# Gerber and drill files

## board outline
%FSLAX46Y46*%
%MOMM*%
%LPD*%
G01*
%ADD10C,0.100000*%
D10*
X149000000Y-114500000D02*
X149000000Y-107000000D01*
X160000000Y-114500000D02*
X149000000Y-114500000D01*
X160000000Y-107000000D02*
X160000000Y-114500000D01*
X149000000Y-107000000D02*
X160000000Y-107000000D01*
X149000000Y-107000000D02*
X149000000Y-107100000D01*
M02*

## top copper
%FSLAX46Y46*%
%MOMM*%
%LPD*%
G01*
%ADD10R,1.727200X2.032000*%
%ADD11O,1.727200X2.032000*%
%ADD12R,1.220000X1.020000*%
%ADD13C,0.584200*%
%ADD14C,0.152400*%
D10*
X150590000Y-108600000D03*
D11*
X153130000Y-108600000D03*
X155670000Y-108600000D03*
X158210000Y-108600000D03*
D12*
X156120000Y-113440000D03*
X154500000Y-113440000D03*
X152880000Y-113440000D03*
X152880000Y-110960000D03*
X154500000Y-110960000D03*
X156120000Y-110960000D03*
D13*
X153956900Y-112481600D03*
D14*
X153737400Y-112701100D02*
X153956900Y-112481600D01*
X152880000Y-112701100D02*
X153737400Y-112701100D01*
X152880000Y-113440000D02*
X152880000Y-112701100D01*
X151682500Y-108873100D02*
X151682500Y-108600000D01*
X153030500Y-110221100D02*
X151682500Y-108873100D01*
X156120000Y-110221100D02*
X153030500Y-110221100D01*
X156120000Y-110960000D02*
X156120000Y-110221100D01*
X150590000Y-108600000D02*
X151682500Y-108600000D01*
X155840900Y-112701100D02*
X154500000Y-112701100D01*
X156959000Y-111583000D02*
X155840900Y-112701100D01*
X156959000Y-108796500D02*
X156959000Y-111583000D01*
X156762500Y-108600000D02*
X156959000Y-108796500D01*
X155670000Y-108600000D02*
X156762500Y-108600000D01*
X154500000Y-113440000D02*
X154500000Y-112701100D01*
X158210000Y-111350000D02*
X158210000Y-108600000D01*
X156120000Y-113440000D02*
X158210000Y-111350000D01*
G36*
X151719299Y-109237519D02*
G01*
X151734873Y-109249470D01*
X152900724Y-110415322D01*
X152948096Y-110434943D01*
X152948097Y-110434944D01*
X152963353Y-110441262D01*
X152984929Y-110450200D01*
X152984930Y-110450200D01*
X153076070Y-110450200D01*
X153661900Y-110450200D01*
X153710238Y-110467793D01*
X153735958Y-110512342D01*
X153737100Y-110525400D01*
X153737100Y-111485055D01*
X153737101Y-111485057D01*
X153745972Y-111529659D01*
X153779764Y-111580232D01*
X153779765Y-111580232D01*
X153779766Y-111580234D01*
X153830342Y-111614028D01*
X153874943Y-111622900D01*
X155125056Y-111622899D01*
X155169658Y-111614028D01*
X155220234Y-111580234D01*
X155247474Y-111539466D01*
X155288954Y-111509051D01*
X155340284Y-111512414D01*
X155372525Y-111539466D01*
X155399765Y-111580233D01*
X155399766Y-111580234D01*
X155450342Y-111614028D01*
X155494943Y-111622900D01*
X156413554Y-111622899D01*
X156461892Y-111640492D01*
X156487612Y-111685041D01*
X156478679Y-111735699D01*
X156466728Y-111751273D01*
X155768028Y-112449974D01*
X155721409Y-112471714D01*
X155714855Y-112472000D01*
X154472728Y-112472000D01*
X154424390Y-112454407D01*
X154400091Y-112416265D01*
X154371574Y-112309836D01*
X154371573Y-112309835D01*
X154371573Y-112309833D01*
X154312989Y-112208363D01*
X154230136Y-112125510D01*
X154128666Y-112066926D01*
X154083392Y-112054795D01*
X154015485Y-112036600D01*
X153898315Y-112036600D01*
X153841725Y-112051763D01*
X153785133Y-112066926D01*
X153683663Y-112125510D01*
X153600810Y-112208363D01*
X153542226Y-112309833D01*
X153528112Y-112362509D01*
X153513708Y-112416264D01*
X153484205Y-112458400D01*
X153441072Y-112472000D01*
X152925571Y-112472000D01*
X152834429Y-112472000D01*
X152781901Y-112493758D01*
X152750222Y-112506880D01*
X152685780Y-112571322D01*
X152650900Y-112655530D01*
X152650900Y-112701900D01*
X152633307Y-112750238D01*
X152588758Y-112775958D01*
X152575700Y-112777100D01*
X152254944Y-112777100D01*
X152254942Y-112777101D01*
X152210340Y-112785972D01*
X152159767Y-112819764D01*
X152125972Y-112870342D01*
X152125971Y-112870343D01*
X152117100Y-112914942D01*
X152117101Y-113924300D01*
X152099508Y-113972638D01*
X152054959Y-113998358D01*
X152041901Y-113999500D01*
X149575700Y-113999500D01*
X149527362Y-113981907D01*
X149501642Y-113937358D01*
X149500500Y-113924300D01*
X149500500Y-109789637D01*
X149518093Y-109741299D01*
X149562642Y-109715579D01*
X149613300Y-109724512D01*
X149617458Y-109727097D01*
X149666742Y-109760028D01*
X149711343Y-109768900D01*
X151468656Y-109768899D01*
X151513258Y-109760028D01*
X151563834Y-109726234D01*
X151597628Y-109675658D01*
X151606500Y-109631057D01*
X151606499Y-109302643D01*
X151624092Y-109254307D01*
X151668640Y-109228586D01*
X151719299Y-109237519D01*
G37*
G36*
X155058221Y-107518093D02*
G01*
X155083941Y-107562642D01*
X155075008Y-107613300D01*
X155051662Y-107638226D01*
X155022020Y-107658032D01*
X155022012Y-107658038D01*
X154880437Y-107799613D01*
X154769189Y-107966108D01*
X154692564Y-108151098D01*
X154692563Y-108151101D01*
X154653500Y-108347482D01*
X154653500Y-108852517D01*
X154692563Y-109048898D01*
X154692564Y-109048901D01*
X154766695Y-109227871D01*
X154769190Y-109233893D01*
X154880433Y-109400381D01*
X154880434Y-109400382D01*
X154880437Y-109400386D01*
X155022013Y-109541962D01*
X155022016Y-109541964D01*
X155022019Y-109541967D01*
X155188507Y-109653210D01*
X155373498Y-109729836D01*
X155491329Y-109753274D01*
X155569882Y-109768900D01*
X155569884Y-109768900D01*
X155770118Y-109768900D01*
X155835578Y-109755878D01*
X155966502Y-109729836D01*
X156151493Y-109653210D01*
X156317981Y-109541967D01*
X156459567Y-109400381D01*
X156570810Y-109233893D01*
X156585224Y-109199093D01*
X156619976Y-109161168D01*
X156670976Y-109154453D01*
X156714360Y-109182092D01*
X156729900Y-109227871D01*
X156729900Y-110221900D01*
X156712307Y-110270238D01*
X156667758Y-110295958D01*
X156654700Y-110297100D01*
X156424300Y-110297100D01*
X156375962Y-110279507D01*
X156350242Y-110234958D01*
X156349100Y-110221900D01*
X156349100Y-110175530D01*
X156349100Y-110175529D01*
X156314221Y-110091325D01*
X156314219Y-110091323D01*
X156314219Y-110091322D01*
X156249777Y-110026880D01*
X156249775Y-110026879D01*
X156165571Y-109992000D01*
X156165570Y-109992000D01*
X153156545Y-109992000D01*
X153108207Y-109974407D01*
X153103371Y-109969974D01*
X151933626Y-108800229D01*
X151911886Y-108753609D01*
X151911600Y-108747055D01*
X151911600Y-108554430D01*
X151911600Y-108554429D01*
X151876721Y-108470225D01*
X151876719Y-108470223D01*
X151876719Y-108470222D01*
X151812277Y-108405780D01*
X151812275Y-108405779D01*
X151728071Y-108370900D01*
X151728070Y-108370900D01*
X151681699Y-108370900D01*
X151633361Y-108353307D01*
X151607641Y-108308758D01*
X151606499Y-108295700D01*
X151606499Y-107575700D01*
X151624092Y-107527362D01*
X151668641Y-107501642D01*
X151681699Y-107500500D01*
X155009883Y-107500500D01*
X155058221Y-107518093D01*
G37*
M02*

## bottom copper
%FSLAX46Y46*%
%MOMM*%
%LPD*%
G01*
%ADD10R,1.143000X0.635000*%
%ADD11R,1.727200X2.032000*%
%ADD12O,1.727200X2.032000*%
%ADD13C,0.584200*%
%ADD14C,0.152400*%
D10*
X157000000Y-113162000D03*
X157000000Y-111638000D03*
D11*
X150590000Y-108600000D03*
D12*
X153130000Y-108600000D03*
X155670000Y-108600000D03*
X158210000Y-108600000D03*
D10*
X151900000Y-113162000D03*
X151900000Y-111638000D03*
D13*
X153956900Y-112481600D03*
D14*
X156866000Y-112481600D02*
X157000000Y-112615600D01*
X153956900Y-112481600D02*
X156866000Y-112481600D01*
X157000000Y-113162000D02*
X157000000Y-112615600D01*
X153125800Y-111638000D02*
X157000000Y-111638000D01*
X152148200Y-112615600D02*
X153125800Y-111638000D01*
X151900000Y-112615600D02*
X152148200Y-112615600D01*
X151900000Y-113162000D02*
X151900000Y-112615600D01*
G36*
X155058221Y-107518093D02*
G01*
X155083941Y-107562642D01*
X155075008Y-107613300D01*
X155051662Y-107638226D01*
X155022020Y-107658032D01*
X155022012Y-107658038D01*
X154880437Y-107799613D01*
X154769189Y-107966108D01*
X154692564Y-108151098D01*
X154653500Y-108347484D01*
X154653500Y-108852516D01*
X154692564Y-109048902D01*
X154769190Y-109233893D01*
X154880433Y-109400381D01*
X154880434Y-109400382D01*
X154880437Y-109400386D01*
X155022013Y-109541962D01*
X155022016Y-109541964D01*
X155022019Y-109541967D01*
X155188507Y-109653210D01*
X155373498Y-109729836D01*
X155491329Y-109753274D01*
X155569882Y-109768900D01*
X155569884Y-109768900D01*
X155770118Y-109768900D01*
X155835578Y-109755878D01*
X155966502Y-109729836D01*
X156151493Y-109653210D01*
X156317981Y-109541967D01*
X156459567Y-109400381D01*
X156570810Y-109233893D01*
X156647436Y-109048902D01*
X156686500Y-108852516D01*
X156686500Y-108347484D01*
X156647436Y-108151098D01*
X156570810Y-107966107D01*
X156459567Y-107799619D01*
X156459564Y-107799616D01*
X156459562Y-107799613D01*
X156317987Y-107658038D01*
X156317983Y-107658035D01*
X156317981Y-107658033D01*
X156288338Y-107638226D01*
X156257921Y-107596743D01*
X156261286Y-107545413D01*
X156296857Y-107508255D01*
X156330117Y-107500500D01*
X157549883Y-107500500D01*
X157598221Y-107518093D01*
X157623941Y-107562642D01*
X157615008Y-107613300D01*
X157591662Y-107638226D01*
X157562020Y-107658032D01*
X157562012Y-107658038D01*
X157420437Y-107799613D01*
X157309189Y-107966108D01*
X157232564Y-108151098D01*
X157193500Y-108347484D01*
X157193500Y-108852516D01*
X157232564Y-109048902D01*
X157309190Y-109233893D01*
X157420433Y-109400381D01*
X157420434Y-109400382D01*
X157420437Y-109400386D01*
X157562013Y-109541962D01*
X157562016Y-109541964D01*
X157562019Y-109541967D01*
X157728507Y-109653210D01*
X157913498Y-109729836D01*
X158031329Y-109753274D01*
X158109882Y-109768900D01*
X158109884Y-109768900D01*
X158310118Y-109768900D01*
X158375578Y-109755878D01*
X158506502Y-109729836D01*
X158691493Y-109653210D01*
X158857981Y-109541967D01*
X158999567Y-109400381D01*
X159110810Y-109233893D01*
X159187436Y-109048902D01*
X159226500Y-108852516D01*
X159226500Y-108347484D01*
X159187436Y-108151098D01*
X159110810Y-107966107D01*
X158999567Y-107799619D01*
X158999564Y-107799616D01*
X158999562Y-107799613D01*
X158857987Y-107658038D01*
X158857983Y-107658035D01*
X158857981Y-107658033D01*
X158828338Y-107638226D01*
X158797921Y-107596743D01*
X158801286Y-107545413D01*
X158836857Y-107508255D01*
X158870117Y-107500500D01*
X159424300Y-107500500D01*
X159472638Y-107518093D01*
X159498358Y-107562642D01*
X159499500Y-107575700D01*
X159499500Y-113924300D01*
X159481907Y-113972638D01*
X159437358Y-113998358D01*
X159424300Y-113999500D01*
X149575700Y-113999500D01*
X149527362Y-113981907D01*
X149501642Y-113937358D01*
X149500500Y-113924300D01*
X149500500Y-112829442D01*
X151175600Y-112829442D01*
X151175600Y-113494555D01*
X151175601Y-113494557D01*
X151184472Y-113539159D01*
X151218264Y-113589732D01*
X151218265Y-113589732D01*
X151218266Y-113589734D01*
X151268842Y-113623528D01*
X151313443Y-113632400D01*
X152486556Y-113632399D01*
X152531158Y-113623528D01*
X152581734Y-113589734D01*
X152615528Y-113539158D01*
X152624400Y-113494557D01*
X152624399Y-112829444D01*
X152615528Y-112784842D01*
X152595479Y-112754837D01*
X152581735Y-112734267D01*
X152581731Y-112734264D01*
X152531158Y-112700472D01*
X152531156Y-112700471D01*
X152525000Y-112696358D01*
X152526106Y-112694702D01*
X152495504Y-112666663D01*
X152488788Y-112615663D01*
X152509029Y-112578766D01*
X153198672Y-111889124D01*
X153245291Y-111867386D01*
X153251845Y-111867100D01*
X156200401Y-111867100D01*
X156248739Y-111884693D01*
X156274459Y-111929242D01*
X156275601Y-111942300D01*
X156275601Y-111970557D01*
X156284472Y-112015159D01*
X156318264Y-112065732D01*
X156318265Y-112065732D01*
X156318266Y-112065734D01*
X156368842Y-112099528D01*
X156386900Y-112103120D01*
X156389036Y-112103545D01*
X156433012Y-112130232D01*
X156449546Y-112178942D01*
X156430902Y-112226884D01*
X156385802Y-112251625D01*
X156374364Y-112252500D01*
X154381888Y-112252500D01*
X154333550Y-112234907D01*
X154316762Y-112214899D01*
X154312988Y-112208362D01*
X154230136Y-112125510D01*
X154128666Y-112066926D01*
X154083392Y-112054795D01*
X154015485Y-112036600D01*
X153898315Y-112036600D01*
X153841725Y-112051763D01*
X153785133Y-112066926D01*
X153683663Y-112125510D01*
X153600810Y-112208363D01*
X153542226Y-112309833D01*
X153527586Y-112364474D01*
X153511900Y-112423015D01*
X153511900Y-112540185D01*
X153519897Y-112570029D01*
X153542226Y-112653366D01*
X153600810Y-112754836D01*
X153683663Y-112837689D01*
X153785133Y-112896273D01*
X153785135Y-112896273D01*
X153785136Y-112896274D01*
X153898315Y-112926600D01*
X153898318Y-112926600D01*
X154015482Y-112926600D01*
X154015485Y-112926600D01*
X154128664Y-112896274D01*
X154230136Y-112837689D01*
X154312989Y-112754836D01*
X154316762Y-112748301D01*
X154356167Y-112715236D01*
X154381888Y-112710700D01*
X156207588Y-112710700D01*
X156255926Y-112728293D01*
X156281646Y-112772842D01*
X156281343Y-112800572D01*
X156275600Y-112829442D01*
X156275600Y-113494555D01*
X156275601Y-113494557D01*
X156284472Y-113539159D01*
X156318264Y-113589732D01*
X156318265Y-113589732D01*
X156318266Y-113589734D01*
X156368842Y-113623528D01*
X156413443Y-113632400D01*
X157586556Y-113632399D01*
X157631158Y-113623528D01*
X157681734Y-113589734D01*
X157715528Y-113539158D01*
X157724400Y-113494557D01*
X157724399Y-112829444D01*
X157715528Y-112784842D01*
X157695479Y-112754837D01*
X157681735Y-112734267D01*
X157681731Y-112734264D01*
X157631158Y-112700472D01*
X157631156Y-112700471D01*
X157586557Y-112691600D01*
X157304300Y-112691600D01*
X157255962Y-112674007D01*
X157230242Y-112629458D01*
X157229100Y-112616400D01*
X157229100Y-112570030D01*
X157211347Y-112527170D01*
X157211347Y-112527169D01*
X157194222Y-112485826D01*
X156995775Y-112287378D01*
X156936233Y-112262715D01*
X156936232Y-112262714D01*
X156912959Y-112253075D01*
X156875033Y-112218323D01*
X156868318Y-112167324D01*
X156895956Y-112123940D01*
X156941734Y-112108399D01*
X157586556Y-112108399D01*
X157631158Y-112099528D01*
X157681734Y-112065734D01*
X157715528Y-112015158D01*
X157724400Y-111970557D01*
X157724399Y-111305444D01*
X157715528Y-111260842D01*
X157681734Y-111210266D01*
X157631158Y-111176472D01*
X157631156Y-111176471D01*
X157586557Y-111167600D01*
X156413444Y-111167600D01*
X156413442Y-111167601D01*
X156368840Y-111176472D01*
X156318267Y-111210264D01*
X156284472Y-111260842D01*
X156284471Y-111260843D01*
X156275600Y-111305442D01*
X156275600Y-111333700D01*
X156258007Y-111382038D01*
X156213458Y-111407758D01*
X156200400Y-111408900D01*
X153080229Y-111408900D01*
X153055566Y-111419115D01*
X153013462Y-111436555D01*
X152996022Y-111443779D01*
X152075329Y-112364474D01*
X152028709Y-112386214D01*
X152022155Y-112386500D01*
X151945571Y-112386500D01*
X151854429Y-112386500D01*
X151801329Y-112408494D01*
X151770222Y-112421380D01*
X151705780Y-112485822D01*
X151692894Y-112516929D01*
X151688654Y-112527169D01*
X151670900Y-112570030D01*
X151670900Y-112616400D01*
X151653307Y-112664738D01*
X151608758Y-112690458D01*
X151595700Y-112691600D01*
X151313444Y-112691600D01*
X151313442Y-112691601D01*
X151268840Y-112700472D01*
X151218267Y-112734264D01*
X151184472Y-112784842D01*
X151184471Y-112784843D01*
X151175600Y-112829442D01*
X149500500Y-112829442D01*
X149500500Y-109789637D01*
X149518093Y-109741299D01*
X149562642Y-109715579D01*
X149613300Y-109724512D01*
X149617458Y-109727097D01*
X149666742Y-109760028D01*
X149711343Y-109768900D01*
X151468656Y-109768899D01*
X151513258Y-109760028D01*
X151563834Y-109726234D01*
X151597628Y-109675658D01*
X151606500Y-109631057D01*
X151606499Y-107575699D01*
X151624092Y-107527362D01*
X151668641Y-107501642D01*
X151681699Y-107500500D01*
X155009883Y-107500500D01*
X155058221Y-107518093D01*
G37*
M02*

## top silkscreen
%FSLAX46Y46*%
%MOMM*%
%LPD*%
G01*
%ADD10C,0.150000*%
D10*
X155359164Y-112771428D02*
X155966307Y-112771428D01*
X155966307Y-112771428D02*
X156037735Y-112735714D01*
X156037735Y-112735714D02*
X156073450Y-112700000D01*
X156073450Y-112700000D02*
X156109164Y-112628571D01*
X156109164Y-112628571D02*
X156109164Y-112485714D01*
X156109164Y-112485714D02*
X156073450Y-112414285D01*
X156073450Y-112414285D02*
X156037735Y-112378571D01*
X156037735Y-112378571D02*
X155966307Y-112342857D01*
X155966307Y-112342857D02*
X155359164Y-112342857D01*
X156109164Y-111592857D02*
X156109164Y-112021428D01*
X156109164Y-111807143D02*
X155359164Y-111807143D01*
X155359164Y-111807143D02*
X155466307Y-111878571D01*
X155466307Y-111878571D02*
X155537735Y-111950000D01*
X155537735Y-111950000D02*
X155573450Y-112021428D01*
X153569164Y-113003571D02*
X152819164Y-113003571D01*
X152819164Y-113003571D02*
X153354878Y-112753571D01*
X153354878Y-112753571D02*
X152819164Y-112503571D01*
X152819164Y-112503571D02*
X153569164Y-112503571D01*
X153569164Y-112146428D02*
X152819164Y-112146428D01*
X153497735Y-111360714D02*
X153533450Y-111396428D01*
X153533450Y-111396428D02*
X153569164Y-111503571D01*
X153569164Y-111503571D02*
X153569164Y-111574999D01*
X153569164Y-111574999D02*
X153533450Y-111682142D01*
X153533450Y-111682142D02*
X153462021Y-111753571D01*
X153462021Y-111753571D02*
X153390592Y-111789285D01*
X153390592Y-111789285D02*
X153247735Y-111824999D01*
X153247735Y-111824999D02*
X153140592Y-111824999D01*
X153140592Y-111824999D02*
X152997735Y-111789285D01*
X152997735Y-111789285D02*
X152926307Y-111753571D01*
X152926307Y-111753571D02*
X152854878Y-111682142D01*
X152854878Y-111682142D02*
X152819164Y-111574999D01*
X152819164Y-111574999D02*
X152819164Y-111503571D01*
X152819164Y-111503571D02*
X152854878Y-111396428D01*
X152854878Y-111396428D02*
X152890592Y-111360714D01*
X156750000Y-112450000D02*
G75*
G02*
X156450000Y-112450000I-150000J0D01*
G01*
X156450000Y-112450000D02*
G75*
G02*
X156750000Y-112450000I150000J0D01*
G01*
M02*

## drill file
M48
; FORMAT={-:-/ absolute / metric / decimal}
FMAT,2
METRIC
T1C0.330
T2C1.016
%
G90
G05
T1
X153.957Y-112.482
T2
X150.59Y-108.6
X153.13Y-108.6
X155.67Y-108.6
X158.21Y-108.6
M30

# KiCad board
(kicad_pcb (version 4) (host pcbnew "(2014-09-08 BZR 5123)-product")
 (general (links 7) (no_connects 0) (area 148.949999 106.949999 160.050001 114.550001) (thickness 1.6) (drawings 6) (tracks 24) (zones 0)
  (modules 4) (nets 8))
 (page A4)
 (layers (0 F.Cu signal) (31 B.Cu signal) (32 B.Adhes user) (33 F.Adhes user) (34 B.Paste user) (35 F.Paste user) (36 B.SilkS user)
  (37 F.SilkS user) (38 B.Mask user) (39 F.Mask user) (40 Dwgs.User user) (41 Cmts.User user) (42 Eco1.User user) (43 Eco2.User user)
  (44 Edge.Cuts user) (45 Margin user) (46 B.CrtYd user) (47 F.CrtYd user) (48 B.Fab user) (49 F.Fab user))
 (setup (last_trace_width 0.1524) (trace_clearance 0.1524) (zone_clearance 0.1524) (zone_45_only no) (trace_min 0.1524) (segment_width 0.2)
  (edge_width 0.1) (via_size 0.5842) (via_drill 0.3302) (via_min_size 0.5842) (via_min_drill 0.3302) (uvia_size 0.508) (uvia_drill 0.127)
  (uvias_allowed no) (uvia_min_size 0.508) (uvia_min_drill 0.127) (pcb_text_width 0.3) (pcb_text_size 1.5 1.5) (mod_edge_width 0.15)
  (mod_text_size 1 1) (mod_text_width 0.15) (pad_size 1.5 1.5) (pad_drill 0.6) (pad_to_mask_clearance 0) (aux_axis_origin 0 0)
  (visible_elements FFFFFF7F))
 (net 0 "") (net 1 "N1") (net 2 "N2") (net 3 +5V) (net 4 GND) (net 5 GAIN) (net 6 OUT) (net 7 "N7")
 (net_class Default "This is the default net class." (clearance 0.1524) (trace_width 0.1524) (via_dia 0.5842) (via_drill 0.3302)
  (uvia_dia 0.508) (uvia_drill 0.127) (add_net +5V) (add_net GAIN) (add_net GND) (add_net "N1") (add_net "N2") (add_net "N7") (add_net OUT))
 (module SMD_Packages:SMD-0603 (layer B.Cu) (at 157 112.4 90)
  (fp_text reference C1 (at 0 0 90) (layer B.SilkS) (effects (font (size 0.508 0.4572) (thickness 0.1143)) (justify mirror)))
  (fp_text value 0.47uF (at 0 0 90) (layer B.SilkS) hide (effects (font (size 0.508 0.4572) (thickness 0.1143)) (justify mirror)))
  (pad 1 smd rect (at -0.762 0 90) (size 0.635 1.143) (layers B.Cu B.Paste B.Mask) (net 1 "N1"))
  (pad 2 smd rect (at 0.762 0 90) (size 0.635 1.143) (layers B.Cu B.Paste B.Mask) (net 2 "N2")))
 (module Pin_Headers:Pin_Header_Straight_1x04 (layer B.Cu) (at 154.4 108.6)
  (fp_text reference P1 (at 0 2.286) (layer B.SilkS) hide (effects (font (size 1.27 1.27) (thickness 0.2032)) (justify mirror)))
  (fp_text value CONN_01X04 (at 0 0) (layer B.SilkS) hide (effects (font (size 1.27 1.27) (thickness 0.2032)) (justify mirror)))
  (pad 1 thru_hole rect (at -3.81 0) (size 1.7272 2.032) (drill 1.016) (layers *.Cu *.Mask B.SilkS) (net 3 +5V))
  (pad 2 thru_hole oval (at -1.27 0) (size 1.7272 2.032) (drill 1.016) (layers *.Cu *.Mask B.SilkS) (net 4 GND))
  (pad 3 thru_hole oval (at 1.27 0) (size 1.7272 2.032) (drill 1.016) (layers *.Cu *.Mask B.SilkS) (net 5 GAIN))
  (pad 4 thru_hole oval (at 3.81 0) (size 1.7272 2.032) (drill 1.016) (layers *.Cu *.Mask B.SilkS) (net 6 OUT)))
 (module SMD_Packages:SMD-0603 (layer B.Cu) (at 151.9 112.4 90)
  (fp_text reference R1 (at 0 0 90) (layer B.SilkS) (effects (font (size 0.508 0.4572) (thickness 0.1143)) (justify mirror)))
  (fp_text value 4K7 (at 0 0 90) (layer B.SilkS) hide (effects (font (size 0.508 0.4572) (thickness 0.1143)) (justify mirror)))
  (pad 1 smd rect (at -0.762 0 90) (size 0.635 1.143) (layers B.Cu B.Paste B.Mask) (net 2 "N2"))
  (pad 2 smd rect (at 0.762 0 90) (size 0.635 1.143) (layers B.Cu B.Paste B.Mask) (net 4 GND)))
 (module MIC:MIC (layer F.Cu) (at 154.5 112.2 270)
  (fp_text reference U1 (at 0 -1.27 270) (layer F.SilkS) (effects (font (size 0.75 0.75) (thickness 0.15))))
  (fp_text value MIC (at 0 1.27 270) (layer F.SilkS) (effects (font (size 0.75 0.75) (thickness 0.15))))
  (fp_circle (center 0.25 -2.1) (end 0.25 -2.25) (layer F.SilkS) (width 0.15))
  (pad 1 smd rect (at 1.24 -1.62 270) (size 1.02 1.22) (layers F.Cu F.Paste F.Mask) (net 6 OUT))
  (pad 2 smd rect (at 1.24 0 270) (size 1.02 1.22) (layers F.Cu F.Paste F.Mask) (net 5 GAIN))
  (pad 3 smd rect (at 1.24 1.62 270) (size 1.02 1.22) (layers F.Cu F.Paste F.Mask) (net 1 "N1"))
  (pad 4 smd rect (at -1.24 1.62 270) (size 1.02 1.22) (layers F.Cu F.Paste F.Mask) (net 4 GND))
  (pad 5 smd rect (at -1.24 0 270) (size 1.02 1.22) (layers F.Cu F.Paste F.Mask) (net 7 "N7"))
  (pad 6 smd rect (at -1.24 -1.62 270) (size 1.02 1.22) (layers F.Cu F.Paste F.Mask) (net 3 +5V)))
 (gr_line (start 149 114.5) (end 149 107) (angle 90) (layer Edge.Cuts) (width 0.1))
 (gr_line (start 160 114.5) (end 149 114.5) (angle 90) (layer Edge.Cuts) (width 0.1))
 (gr_line (start 160 107) (end 160 114.5) (angle 90) (layer Edge.Cuts) (width 0.1))
 (gr_line (start 149 107) (end 160 107) (angle 90) (layer Edge.Cuts) (width 0.1))
 (gr_line (start 149 107) (end 149 107.1) (angle 90) (layer Edge.Cuts) (width 0.1))
 (via (at 153.9569 112.4816) (size 0.5842) (layers F.Cu B.Cu) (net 1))
 (segment (start 153.7374 112.7011) (end 153.9569 112.4816) (width 0.1524) (layer F.Cu) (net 1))
 (segment (start 152.88 112.7011) (end 153.7374 112.7011) (width 0.1524) (layer F.Cu) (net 1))
 (segment (start 156.866 112.4816) (end 157 112.6156) (width 0.1524) (layer B.Cu) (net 1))
 (segment (start 153.9569 112.4816) (end 156.866 112.4816) (width 0.1524) (layer B.Cu) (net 1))
 (segment (start 152.88 113.44) (end 152.88 112.7011) (width 0.1524) (layer F.Cu) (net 1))
 (segment (start 157 113.162) (end 157 112.6156) (width 0.1524) (layer B.Cu) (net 1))
 (segment (start 153.1258 111.638) (end 157 111.638) (width 0.1524) (layer B.Cu) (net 2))
 (segment (start 152.1482 112.6156) (end 153.1258 111.638) (width 0.1524) (layer B.Cu) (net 2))
 (segment (start 151.9 112.6156) (end 152.1482 112.6156) (width 0.1524) (layer B.Cu) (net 2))
 (segment (start 151.9 113.162) (end 151.9 112.6156) (width 0.1524) (layer B.Cu) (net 2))
 (segment (start 151.6825 108.8731) (end 151.6825 108.6) (width 0.1524) (layer F.Cu) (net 3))
 (segment (start 153.0305 110.2211) (end 151.6825 108.8731) (width 0.1524) (layer F.Cu) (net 3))
 (segment (start 156.12 110.2211) (end 153.0305 110.2211) (width 0.1524) (layer F.Cu) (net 3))
 (segment (start 156.12 110.96) (end 156.12 110.2211) (width 0.1524) (layer F.Cu) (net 3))
 (segment (start 150.59 108.6) (end 151.6825 108.6) (width 0.1524) (layer F.Cu) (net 3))
 (segment (start 155.8409 112.7011) (end 154.5 112.7011) (width 0.1524) (layer F.Cu) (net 5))
 (segment (start 156.959 111.583) (end 155.8409 112.7011) (width 0.1524) (layer F.Cu) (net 5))
 (segment (start 156.959 108.7965) (end 156.959 111.583) (width 0.1524) (layer F.Cu) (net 5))
 (segment (start 156.7625 108.6) (end 156.959 108.7965) (width 0.1524) (layer F.Cu) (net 5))
 (segment (start 155.67 108.6) (end 156.7625 108.6) (width 0.1524) (layer F.Cu) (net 5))
 (segment (start 154.5 113.44) (end 154.5 112.7011) (width 0.1524) (layer F.Cu) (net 5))
 (segment (start 158.21 111.35) (end 158.21 108.6) (width 0.1524) (layer F.Cu) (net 6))
 (segment (start 156.12 113.44) (end 158.21 111.35) (width 0.1524) (layer F.Cu) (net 6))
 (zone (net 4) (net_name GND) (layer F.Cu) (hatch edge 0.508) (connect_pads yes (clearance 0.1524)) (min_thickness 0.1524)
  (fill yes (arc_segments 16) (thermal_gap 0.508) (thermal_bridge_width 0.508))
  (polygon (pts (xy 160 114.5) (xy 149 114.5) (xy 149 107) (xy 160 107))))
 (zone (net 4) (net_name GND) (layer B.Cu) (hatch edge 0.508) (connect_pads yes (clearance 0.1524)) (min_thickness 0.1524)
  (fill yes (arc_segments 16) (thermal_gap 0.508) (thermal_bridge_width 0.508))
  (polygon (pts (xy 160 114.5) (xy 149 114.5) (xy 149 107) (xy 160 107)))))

